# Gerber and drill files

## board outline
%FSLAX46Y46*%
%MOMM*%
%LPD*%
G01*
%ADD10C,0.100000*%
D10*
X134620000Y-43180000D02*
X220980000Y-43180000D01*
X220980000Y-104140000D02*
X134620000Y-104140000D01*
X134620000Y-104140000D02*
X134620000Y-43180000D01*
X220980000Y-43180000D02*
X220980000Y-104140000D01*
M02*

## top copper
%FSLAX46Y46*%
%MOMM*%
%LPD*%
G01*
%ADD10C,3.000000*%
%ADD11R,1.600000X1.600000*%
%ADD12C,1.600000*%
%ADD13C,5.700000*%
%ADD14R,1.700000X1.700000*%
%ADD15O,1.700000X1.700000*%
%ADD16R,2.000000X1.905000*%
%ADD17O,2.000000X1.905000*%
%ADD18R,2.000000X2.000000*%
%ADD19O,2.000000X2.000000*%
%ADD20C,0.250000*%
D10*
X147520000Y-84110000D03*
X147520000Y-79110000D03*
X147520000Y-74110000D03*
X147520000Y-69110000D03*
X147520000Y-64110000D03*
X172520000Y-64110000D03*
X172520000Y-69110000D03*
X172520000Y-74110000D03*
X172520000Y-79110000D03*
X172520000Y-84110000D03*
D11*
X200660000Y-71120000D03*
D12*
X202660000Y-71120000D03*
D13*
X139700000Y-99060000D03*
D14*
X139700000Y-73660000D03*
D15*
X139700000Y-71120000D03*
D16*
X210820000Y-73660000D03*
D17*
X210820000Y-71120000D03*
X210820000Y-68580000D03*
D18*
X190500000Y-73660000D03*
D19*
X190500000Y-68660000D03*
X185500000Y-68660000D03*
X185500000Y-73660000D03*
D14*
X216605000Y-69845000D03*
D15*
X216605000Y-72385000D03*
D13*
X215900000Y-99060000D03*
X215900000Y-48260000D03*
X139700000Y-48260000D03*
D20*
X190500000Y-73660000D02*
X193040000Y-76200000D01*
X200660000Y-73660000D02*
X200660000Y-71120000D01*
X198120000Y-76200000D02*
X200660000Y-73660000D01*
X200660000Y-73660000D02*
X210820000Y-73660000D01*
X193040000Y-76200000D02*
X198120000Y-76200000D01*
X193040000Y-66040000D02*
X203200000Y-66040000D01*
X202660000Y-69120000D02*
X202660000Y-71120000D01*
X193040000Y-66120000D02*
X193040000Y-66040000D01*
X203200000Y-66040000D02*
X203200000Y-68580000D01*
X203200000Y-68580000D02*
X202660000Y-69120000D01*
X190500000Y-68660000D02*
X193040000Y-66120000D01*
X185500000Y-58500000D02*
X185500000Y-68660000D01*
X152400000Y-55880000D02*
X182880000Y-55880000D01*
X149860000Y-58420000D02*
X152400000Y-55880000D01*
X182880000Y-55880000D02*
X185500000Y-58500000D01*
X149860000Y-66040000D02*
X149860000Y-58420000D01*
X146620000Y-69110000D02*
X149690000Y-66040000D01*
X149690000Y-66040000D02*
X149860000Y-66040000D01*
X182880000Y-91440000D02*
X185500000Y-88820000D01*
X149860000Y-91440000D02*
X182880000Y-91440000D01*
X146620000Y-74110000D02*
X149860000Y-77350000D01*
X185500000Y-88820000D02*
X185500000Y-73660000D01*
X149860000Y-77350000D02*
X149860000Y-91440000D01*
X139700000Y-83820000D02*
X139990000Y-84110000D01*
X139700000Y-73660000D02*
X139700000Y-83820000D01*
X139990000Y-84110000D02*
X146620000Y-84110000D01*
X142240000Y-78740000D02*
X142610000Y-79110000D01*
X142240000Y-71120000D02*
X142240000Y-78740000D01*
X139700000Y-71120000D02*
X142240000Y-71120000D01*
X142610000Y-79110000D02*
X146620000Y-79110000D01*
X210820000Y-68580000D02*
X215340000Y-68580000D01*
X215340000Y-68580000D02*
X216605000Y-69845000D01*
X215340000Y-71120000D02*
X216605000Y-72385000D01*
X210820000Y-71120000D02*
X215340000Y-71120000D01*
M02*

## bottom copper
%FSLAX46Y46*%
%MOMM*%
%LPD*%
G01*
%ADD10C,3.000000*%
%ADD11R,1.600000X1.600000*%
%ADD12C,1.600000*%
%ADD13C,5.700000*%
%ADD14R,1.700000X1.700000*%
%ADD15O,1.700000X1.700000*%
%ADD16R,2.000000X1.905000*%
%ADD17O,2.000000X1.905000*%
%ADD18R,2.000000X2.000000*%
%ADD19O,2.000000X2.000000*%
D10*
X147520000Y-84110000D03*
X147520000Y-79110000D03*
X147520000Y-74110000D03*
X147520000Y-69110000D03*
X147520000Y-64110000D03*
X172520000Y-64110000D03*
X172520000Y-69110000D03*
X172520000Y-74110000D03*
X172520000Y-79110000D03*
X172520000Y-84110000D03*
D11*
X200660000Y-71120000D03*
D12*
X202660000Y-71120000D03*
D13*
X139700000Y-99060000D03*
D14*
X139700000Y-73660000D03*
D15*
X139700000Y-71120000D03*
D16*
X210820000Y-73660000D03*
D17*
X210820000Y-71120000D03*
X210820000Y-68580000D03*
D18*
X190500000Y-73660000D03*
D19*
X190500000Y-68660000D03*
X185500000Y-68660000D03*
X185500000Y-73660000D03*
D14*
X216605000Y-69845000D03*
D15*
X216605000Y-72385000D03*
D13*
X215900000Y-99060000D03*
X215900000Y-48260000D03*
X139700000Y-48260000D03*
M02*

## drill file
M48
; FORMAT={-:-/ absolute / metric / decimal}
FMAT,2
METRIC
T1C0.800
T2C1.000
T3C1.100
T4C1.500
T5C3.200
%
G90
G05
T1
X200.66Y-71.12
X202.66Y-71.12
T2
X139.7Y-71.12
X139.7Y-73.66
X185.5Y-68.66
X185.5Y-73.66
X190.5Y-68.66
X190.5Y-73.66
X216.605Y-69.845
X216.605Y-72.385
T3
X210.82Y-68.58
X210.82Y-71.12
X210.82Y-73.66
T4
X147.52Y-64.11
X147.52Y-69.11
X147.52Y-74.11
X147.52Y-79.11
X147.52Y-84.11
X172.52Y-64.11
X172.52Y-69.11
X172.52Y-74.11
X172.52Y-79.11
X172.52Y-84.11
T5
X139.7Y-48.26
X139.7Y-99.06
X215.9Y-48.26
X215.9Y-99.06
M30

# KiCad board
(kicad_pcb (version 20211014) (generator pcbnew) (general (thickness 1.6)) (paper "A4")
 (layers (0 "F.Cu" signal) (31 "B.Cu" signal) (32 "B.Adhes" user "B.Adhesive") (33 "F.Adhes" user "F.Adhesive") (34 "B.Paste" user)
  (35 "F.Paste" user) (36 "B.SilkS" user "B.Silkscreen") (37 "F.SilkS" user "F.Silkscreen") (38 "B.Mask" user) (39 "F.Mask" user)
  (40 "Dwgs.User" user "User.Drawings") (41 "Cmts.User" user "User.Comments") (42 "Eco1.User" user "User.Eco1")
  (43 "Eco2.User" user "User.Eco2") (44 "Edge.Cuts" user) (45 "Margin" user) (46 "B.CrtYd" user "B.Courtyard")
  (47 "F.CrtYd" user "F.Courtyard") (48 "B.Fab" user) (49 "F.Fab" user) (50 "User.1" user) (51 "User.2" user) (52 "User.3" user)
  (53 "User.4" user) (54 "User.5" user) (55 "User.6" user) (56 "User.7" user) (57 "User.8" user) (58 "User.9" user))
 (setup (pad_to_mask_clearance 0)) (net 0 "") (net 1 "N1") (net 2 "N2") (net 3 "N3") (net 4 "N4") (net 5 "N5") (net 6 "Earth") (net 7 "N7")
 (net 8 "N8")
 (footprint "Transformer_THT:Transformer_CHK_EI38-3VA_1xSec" (layer "F.Cu") (at 147.52 84.11)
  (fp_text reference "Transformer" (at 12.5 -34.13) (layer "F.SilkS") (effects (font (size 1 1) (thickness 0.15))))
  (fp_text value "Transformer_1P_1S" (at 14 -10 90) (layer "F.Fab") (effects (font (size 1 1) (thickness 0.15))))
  (pad "1" thru_hole circle (at 0 0) (size 3 3) (drill 1.5) (layers *.Cu *.Mask) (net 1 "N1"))
  (pad "2" thru_hole circle (at 0 -5) (size 3 3) (drill 1.5) (layers *.Cu *.Mask) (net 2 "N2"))
  (pad "3" thru_hole circle (at 0 -10) (size 3 3) (drill 1.5) (layers *.Cu *.Mask) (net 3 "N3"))
  (pad "4" thru_hole circle (at 0 -15) (size 3 3) (drill 1.5) (layers *.Cu *.Mask) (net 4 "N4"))
  (pad "5" thru_hole circle (at 0 -20) (size 3 3) (drill 1.5) (layers *.Cu *.Mask))
  (pad "6" thru_hole circle (at 25 -20) (size 3 3) (drill 1.5) (layers *.Cu *.Mask))
  (pad "7" thru_hole circle (at 25 -15) (size 3 3) (drill 1.5) (layers *.Cu *.Mask))
  (pad "8" thru_hole circle (at 25 -10) (size 3 3) (drill 1.5) (layers *.Cu *.Mask))
  (pad "9" thru_hole circle (at 25 -5) (size 3 3) (drill 1.5) (layers *.Cu *.Mask))
  (pad "10" thru_hole circle (at 25 0) (size 3 3) (drill 1.5) (layers *.Cu *.Mask)))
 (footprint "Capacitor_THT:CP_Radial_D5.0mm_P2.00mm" (layer "F.Cu") (at 200.66 71.12)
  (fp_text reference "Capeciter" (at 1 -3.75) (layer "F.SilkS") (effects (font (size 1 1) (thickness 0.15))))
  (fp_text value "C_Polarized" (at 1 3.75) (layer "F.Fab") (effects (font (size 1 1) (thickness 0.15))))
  (pad "1" thru_hole rect (at 0 0) (size 1.6 1.6) (drill 0.8) (layers *.Cu *.Mask) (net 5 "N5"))
  (pad "2" thru_hole circle (at 2 0) (size 1.6 1.6) (drill 0.8) (layers *.Cu *.Mask) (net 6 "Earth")))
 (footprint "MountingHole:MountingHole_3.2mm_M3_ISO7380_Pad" (layer "F.Cu") (at 139.7 99.06)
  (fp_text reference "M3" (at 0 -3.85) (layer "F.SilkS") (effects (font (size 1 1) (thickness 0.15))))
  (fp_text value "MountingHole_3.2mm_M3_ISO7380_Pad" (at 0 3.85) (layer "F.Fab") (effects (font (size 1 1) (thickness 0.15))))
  (pad "1" thru_hole circle (at 0 0) (size 5.7 5.7) (drill 3.2) (layers *.Cu *.Mask)))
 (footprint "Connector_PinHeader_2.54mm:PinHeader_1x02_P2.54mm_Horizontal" (layer "F.Cu") (at 139.7 73.66 180)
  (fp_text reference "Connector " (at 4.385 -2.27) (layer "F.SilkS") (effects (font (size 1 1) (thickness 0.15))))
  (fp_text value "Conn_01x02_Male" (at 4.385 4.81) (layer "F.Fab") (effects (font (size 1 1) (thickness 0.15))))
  (pad "1" thru_hole rect (at 0 0 180) (size 1.7 1.7) (drill 1) (layers *.Cu *.Mask) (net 1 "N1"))
  (pad "2" thru_hole oval (at 0 2.54 180) (size 1.7 1.7) (drill 1) (layers *.Cu *.Mask) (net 2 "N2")))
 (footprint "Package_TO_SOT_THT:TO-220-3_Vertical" (layer "F.Cu") (at 210.82 73.66 90)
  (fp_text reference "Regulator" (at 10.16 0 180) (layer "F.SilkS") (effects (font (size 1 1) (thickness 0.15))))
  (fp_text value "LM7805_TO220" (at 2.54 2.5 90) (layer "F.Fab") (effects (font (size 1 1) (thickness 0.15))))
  (pad "1" thru_hole rect (at 0 0 90) (size 1.905 2) (drill 1.1) (layers *.Cu *.Mask) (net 5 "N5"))
  (pad "2" thru_hole oval (at 2.54 0 90) (size 1.905 2) (drill 1.1) (layers *.Cu *.Mask) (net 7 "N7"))
  (pad "3" thru_hole oval (at 5.08 0 90) (size 1.905 2) (drill 1.1) (layers *.Cu *.Mask) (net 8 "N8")))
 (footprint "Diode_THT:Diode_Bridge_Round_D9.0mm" (layer "F.Cu") (at 190.5 73.66 180)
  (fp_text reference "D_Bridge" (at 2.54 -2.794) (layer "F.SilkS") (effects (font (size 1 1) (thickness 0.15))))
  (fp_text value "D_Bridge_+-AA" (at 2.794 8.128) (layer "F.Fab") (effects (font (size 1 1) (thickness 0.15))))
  (pad "1" thru_hole rect (at 0 0 180) (size 2 2) (drill 1) (layers *.Cu *.Mask) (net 5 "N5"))
  (pad "2" thru_hole oval (at 0 5 180) (size 2 2) (drill 1) (layers *.Cu *.Mask) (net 6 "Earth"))
  (pad "3" thru_hole oval (at 5 5 180) (size 2 2) (drill 1) (layers *.Cu *.Mask) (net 4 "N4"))
  (pad "4" thru_hole oval (at 5 0 180) (size 2 2) (drill 1) (layers *.Cu *.Mask) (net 3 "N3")))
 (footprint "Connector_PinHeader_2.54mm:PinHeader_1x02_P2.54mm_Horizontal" (layer "F.Cu") (at 216.605 69.845)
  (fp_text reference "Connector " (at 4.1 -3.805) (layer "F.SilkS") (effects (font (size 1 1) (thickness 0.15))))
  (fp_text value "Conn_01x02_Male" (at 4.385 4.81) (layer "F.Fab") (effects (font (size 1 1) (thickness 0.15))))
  (pad "1" thru_hole rect (at 0 0) (size 1.7 1.7) (drill 1) (layers *.Cu *.Mask) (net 8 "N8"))
  (pad "2" thru_hole oval (at 0 2.54) (size 1.7 1.7) (drill 1) (layers *.Cu *.Mask) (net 7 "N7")))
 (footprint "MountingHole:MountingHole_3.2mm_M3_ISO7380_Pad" (layer "F.Cu") (at 215.9 99.06)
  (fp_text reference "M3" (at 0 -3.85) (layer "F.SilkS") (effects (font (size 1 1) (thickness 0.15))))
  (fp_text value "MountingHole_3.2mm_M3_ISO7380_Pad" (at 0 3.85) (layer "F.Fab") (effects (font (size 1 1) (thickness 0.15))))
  (pad "1" thru_hole circle (at 0 0) (size 5.7 5.7) (drill 3.2) (layers *.Cu *.Mask)))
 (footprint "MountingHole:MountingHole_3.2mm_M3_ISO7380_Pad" (layer "F.Cu") (at 215.9 48.26)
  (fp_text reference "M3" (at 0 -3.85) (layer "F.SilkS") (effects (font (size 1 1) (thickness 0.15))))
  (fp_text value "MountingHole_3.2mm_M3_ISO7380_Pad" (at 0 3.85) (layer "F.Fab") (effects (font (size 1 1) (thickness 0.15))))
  (pad "1" thru_hole circle (at 0 0) (size 5.7 5.7) (drill 3.2) (layers *.Cu *.Mask)))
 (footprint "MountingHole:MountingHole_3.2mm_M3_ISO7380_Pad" (layer "F.Cu") (at 139.7 48.26)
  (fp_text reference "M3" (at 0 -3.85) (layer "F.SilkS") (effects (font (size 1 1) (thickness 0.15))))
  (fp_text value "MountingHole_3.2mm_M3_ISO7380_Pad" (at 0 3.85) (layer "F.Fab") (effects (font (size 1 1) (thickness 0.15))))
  (pad "1" thru_hole circle (at 0 0) (size 5.7 5.7) (drill 3.2) (layers *.Cu *.Mask)))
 (gr_line (start 134.62 43.18) (end 220.98 43.18) (layer "Edge.Cuts") (width 0.1))
 (gr_line (start 220.98 104.14) (end 134.62 104.14) (layer "Edge.Cuts") (width 0.1))
 (gr_line (start 134.62 104.14) (end 134.62 43.18) (layer "Edge.Cuts") (width 0.1))
 (gr_line (start 220.98 43.18) (end 220.98 104.14) (layer "Edge.Cuts") (width 0.1))
 (segment (start 190.5 73.66) (end 193.04 76.2) (width 0.25) (layer "F.Cu") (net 5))
 (segment (start 200.66 73.66) (end 200.66 71.12) (width 0.25) (layer "F.Cu") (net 5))
 (segment (start 198.12 76.2) (end 200.66 73.66) (width 0.25) (layer "F.Cu") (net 5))
 (segment (start 200.66 73.66) (end 210.82 73.66) (width 0.25) (layer "F.Cu") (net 5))
 (segment (start 193.04 76.2) (end 198.12 76.2) (width 0.25) (layer "F.Cu") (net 5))
 (segment (start 193.04 66.04) (end 203.2 66.04) (width 0.25) (layer "F.Cu") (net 6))
 (segment (start 202.66 69.12) (end 202.66 71.12) (width 0.25) (layer "F.Cu") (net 6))
 (segment (start 193.04 66.12) (end 193.04 66.04) (width 0.25) (layer "F.Cu") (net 6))
 (segment (start 203.2 66.04) (end 203.2 68.58) (width 0.25) (layer "F.Cu") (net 6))
 (segment (start 203.2 68.58) (end 202.66 69.12) (width 0.25) (layer "F.Cu") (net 6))
 (segment (start 190.5 68.66) (end 193.04 66.12) (width 0.25) (layer "F.Cu") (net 6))
 (segment (start 185.5 58.5) (end 185.5 68.66) (width 0.25) (layer "F.Cu") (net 4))
 (segment (start 152.4 55.88) (end 182.88 55.88) (width 0.25) (layer "F.Cu") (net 4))
 (segment (start 149.86 58.42) (end 152.4 55.88) (width 0.25) (layer "F.Cu") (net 4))
 (segment (start 182.88 55.88) (end 185.5 58.5) (width 0.25) (layer "F.Cu") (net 4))
 (segment (start 149.86 66.04) (end 149.86 58.42) (width 0.25) (layer "F.Cu") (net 4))
 (segment (start 146.62 69.11) (end 149.69 66.04) (width 0.25) (layer "F.Cu") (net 4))
 (segment (start 149.69 66.04) (end 149.86 66.04) (width 0.25) (layer "F.Cu") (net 4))
 (segment (start 182.88 91.44) (end 185.5 88.82) (width 0.25) (layer "F.Cu") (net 3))
 (segment (start 149.86 91.44) (end 182.88 91.44) (width 0.25) (layer "F.Cu") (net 3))
 (segment (start 146.62 74.11) (end 149.86 77.35) (width 0.25) (layer "F.Cu") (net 3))
 (segment (start 185.5 88.82) (end 185.5 73.66) (width 0.25) (layer "F.Cu") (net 3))
 (segment (start 149.86 77.35) (end 149.86 91.44) (width 0.25) (layer "F.Cu") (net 3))
 (segment (start 139.7 83.82) (end 139.99 84.11) (width 0.25) (layer "F.Cu") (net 1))
 (segment (start 139.7 73.66) (end 139.7 83.82) (width 0.25) (layer "F.Cu") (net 1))
 (segment (start 139.99 84.11) (end 146.62 84.11) (width 0.25) (layer "F.Cu") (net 1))
 (segment (start 142.24 78.74) (end 142.61 79.11) (width 0.25) (layer "F.Cu") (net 2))
 (segment (start 142.24 71.12) (end 142.24 78.74) (width 0.25) (layer "F.Cu") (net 2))
 (segment (start 139.7 71.12) (end 142.24 71.12) (width 0.25) (layer "F.Cu") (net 2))
 (segment (start 142.61 79.11) (end 146.62 79.11) (width 0.25) (layer "F.Cu") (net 2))
 (segment (start 210.82 68.58) (end 215.34 68.58) (width 0.25) (layer "F.Cu") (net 8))
 (segment (start 215.34 68.58) (end 216.605 69.845) (width 0.25) (layer "F.Cu") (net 8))
 (segment (start 215.34 71.12) (end 216.605 72.385) (width 0.25) (layer "F.Cu") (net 7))
 (segment (start 210.82 71.12) (end 215.34 71.12) (width 0.25) (layer "F.Cu") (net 7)))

